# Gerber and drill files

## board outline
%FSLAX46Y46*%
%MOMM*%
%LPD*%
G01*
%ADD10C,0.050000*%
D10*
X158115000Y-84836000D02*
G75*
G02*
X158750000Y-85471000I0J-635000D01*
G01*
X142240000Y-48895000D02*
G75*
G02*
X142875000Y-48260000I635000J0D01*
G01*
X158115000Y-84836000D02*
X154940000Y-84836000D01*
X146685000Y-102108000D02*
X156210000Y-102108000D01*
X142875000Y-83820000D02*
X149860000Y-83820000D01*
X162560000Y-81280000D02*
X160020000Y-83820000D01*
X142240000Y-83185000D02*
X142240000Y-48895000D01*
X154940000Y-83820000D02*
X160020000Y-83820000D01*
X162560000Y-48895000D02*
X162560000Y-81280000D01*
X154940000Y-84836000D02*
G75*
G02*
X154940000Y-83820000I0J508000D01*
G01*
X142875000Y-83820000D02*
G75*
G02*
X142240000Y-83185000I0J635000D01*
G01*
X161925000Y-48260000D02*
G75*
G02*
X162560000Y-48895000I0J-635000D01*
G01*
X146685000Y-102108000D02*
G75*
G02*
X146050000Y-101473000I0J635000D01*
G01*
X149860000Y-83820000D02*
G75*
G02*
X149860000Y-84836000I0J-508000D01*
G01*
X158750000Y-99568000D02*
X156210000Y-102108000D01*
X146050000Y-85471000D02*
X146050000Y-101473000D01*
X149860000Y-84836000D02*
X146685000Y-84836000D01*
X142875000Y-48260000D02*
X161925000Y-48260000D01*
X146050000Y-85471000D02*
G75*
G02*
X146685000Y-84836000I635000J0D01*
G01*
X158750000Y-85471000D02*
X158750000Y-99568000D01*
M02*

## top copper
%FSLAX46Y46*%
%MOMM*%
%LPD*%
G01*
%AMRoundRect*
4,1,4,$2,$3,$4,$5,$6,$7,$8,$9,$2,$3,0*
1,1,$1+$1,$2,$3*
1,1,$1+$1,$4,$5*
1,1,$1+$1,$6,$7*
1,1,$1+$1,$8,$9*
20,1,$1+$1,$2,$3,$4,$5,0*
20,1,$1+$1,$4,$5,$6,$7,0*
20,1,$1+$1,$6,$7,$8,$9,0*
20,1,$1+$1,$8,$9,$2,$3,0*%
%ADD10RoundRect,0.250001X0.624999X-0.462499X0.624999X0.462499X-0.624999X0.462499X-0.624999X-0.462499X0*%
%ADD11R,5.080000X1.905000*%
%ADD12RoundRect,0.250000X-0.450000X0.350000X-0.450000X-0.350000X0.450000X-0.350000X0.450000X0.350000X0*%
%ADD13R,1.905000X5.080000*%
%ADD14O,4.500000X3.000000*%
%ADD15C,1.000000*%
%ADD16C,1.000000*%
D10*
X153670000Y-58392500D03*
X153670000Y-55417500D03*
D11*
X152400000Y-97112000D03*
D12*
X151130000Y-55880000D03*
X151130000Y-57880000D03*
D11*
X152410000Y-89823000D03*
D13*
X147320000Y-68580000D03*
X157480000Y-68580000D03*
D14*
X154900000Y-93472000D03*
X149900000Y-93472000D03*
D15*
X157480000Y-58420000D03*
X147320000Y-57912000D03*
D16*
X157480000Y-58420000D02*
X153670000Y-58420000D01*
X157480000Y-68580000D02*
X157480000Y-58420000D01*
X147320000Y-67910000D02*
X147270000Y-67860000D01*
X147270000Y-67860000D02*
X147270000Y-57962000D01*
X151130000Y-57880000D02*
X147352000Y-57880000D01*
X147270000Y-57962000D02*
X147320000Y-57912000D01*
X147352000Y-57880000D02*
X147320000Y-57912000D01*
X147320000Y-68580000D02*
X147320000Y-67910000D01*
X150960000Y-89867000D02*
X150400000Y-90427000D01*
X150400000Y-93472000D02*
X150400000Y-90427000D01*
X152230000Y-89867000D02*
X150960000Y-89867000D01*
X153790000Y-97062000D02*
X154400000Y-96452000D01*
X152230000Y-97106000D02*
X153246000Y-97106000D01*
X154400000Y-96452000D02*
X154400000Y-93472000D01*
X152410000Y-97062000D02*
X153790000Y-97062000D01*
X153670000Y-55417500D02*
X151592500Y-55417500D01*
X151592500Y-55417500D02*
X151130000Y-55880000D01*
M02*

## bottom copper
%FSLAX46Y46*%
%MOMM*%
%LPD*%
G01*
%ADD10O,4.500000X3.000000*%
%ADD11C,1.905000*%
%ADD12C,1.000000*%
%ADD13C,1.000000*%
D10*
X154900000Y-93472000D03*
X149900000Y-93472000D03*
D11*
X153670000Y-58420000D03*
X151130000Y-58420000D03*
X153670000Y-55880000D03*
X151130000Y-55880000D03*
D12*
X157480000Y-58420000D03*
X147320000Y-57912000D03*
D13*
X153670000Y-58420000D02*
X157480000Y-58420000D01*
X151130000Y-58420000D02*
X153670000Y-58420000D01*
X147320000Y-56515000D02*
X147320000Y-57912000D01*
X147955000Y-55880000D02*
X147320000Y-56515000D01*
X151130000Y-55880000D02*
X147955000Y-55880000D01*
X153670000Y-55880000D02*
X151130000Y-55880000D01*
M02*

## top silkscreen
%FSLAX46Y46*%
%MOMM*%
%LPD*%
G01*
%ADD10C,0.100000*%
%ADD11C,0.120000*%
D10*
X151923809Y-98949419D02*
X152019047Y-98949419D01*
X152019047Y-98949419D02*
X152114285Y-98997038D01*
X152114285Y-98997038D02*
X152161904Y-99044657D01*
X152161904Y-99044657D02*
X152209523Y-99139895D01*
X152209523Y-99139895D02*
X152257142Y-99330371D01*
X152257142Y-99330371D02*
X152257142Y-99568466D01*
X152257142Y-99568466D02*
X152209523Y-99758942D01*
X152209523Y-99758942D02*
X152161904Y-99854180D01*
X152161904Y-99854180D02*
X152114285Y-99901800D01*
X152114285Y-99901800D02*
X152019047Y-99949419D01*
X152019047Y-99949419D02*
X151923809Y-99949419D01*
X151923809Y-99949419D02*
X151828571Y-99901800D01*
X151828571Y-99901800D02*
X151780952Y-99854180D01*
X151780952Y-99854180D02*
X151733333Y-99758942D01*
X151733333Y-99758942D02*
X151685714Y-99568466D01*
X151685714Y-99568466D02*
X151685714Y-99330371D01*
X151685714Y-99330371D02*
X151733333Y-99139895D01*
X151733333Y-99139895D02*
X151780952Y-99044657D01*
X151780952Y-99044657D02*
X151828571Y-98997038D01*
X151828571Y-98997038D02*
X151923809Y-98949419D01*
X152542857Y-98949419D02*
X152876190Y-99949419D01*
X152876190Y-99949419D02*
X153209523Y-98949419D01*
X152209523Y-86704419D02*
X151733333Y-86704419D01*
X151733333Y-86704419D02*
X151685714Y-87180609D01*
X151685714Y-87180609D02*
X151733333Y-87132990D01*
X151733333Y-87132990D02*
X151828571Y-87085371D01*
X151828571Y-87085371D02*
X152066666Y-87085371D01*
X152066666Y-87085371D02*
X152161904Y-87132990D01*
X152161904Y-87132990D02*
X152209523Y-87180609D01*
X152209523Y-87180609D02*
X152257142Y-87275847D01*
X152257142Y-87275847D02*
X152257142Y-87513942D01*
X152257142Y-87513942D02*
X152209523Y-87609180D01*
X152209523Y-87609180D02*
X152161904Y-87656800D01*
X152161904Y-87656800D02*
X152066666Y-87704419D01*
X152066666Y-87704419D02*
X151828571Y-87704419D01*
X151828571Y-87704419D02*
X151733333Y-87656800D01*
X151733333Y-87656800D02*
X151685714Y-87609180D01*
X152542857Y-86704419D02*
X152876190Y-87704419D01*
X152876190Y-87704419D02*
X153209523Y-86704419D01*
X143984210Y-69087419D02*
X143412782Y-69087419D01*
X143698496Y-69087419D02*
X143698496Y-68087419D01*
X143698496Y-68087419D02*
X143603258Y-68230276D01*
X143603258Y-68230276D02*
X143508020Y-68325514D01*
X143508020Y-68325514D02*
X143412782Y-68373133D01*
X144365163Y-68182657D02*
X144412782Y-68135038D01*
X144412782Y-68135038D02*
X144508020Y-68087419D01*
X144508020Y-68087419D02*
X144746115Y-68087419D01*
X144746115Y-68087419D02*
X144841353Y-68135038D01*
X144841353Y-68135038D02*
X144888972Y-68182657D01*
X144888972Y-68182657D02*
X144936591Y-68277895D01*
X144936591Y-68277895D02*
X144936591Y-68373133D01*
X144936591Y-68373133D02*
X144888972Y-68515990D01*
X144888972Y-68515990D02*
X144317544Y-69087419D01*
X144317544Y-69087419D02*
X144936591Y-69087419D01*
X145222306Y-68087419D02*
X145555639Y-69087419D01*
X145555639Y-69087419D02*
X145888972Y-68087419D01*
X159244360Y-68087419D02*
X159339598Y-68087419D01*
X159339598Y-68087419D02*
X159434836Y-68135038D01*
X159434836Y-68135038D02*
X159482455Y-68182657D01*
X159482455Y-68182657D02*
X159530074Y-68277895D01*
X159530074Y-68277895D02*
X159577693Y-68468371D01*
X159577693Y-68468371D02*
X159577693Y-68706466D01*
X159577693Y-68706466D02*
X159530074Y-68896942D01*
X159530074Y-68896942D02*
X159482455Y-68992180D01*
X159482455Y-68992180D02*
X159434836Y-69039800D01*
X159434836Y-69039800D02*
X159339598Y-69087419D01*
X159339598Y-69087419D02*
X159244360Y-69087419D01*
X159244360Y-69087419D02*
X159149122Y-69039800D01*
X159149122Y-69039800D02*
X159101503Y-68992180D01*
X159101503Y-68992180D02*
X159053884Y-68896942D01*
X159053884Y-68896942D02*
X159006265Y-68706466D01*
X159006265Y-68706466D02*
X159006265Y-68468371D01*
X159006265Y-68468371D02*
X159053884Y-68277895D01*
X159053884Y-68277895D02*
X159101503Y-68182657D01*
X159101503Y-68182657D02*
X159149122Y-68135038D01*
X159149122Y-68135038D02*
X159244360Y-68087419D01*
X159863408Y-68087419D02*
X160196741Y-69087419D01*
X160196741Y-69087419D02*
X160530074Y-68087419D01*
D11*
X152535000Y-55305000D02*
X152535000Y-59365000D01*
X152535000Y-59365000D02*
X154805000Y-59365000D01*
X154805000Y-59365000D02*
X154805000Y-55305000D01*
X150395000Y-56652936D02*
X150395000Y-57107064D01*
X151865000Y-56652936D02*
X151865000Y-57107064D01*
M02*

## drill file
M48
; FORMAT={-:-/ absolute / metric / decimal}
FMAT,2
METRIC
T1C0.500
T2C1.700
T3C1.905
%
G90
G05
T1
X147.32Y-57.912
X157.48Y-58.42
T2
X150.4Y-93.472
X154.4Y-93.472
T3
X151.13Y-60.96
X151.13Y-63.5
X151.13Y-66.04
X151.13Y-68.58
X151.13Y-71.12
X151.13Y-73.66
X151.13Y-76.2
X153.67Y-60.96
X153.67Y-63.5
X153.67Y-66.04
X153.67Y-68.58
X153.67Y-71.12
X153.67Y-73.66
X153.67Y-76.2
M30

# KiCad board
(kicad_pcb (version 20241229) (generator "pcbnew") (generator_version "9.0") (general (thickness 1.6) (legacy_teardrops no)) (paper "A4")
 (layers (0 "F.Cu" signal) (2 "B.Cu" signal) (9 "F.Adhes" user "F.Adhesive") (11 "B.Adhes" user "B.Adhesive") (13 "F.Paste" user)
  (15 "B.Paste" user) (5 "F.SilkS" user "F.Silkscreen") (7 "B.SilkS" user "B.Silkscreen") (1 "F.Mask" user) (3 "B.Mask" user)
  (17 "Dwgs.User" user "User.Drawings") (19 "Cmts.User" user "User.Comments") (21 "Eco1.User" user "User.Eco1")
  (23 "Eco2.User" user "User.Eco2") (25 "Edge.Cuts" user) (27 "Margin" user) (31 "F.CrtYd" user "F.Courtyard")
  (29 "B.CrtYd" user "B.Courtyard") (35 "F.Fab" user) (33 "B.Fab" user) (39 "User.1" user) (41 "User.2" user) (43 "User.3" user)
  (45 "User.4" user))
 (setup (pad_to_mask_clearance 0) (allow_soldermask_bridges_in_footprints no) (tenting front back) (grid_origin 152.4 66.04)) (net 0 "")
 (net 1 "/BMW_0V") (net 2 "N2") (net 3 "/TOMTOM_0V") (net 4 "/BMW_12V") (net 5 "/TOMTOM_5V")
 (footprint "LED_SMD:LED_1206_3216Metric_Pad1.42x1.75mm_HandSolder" (layer "F.Cu") (at 153.67 56.905 90)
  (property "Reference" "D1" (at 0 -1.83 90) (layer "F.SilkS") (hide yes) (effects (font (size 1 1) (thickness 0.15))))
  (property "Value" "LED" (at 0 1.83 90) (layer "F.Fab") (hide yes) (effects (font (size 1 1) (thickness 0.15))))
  (fp_line (start 1.6 -1.135) (end -2.46 -1.135) (stroke (width 0.12) (type solid)) (layer "F.SilkS"))
  (fp_line (start -2.46 -1.135) (end -2.46 1.135) (stroke (width 0.12) (type solid)) (layer "F.SilkS"))
  (fp_line (start -2.46 1.135) (end 1.6 1.135) (stroke (width 0.12) (type solid)) (layer "F.SilkS"))
  (pad "1" smd roundrect (at -1.4875 0 90) (size 1.425 1.75) (layers "F.Cu" "F.Mask" "F.Paste") (roundrect_rratio 0.175439)
   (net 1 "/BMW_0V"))
  (pad "2" smd roundrect (at 1.4875 0 90) (size 1.425 1.75) (layers "F.Cu" "F.Mask" "F.Paste") (roundrect_rratio 0.175439) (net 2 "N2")))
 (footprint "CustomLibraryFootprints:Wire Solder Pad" (layer "F.Cu") (at 152.4 97.112 -90)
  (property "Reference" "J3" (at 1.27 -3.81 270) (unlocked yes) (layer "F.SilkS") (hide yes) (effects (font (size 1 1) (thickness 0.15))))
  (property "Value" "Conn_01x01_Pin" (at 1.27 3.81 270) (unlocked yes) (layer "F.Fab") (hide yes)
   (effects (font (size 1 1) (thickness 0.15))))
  (pad "1" smd rect (at 0 0 270) (size 1.905 5.08) (layers "F.Cu" "F.Mask" "F.Paste") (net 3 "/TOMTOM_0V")))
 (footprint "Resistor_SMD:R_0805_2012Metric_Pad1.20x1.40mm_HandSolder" (layer "F.Cu") (at 151.13 56.88 -90)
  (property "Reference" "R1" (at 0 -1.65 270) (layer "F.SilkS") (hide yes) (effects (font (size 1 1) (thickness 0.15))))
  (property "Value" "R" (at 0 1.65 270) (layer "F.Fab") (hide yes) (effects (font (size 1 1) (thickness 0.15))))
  (fp_line (start -0.227064 0.735) (end 0.227064 0.735) (stroke (width 0.12) (type solid)) (layer "F.SilkS"))
  (fp_line (start -0.227064 -0.735) (end 0.227064 -0.735) (stroke (width 0.12) (type solid)) (layer "F.SilkS"))
  (pad "1" smd roundrect (at -1 0 270) (size 1.2 1.4) (layers "F.Cu" "F.Mask" "F.Paste") (roundrect_rratio 0.208333) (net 2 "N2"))
  (pad "2" smd roundrect (at 1 0 270) (size 1.2 1.4) (layers "F.Cu" "F.Mask" "F.Paste") (roundrect_rratio 0.208333) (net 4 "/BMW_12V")))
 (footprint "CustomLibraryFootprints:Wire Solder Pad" (layer "F.Cu") (at 152.41 89.823 -90)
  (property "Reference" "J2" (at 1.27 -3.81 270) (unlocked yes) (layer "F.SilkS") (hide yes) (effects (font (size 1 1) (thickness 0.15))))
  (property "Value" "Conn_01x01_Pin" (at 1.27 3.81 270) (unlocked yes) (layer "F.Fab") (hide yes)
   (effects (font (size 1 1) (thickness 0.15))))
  (pad "1" smd rect (at 0 0 270) (size 1.905 5.08) (layers "F.Cu" "F.Mask" "F.Paste") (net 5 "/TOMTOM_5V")))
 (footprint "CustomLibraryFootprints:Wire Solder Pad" (layer "F.Cu") (at 147.32 68.58 180)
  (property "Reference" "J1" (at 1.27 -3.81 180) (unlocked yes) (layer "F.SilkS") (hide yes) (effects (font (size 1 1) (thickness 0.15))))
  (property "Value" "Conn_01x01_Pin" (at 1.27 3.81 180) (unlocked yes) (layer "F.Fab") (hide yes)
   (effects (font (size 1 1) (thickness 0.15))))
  (pad "1" smd rect (at 0 0 180) (size 1.905 5.08) (layers "F.Cu" "F.Mask" "F.Paste") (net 4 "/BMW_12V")))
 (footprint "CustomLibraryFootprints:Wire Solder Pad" (layer "F.Cu") (at 157.48 68.58 180)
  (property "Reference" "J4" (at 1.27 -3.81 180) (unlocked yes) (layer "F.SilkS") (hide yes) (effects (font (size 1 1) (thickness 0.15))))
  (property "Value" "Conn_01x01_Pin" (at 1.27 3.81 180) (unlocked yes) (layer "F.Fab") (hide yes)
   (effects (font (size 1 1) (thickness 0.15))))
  (pad "1" smd rect (at 0 0 180) (size 1.905 5.08) (layers "F.Cu" "F.Mask" "F.Paste") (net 1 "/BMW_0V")))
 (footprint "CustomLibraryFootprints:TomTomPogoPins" (layer "F.Cu") (at 154.4 93.472 180)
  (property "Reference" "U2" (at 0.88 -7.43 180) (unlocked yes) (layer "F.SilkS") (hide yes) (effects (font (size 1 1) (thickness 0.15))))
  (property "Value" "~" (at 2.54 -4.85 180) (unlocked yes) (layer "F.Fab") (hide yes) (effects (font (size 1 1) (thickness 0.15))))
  (pad "1" thru_hole oval (at 0 0 180) (size 4.5 3) (drill 1.7 (offset -0.5 0)) (layers "*.Cu" "*.Mask") (remove_unused_layers no)
   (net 3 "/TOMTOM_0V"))
  (pad "2" thru_hole oval (at 4 0 180) (size 4.5 3) (drill 1.7 (offset 0.5 0)) (layers "*.Cu" "*.Mask") (remove_unused_layers no)
   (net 5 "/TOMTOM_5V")))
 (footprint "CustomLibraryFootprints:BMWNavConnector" (layer "B.Cu") (at 151.13 76.2 180)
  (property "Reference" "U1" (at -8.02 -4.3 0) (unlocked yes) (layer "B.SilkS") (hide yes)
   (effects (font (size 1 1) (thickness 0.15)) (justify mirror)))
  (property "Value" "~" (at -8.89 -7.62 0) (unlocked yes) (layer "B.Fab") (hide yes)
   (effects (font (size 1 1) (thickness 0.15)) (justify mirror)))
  (pad "" np_thru_hole circle (at -2.54 0 180) (size 1.905 1.905) (drill 1.905) (layers "*.Cu" "*.Mask"))
  (pad "" np_thru_hole circle (at -2.54 2.54 180) (size 1.905 1.905) (drill 1.905) (layers "*.Cu" "*.Mask"))
  (pad "" np_thru_hole circle (at -2.54 5.08 180) (size 1.905 1.905) (drill 1.905) (layers "*.Cu" "*.Mask"))
  (pad "" np_thru_hole circle (at -2.54 7.62 180) (size 1.905 1.905) (drill 1.905) (layers "*.Cu" "*.Mask"))
  (pad "" np_thru_hole circle (at -2.54 10.16 180) (size 1.905 1.905) (drill 1.905) (layers "*.Cu" "*.Mask"))
  (pad "" np_thru_hole circle (at -2.54 12.7 180) (size 1.905 1.905) (drill 1.905) (layers "*.Cu" "*.Mask"))
  (pad "" np_thru_hole circle (at -2.54 15.24 180) (size 1.905 1.905) (drill 1.905) (layers "*.Cu" "*.Mask"))
  (pad "" np_thru_hole circle (at 0 0 180) (size 1.905 1.905) (drill 1.905) (layers "*.Cu" "*.Mask"))
  (pad "" np_thru_hole circle (at 0 2.54 180) (size 1.905 1.905) (drill 1.905) (layers "*.Cu" "*.Mask"))
  (pad "" np_thru_hole circle (at 0 5.08 180) (size 1.905 1.905) (drill 1.905) (layers "*.Cu" "*.Mask"))
  (pad "" np_thru_hole circle (at 0 7.62 180) (size 1.905 1.905) (drill 1.905) (layers "*.Cu" "*.Mask"))
  (pad "" np_thru_hole circle (at 0 10.16 180) (size 1.905 1.905) (drill 1.905) (layers "*.Cu" "*.Mask"))
  (pad "" np_thru_hole circle (at 0 12.7 180) (size 1.905 1.905) (drill 1.905) (layers "*.Cu" "*.Mask"))
  (pad "" np_thru_hole circle (at 0 15.24 180) (size 1.905 1.905) (drill 1.905) (layers "*.Cu" "*.Mask"))
  (pad "15" smd circle (at -2.54 17.78 180) (size 1.905 1.905) (layers "B.Cu" "B.Mask" "B.Paste") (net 1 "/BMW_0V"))
  (pad "16" smd circle (at 0 17.78 180) (size 1.905 1.905) (layers "B.Cu" "B.Mask" "B.Paste") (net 1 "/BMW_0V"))
  (pad "17" smd circle (at -2.54 20.32 180) (size 1.905 1.905) (layers "B.Cu" "B.Mask" "B.Paste") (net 4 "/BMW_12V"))
  (pad "18" smd circle (at 0 20.32 180) (size 1.905 1.905) (layers "B.Cu" "B.Mask" "B.Paste") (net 4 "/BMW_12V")))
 (gr_arc (start 158.115 84.836) (mid 158.564013 85.021987) (end 158.75 85.471) (stroke (width 0.05) (type default)) (layer "Edge.Cuts"))
 (gr_arc (start 142.24 48.895) (mid 142.425987 48.445987) (end 142.875 48.26) (stroke (width 0.05) (type default)) (layer "Edge.Cuts"))
 (gr_line (start 158.115 84.836) (end 154.94 84.836) (stroke (width 0.05) (type default)) (layer "Edge.Cuts"))
 (gr_line (start 146.685 102.108) (end 156.21 102.108) (stroke (width 0.05) (type default)) (layer "Edge.Cuts"))
 (gr_line (start 142.875 83.82) (end 149.86 83.82) (stroke (width 0.05) (type default)) (layer "Edge.Cuts"))
 (gr_line (start 162.56 81.28) (end 160.02 83.82) (stroke (width 0.05) (type default)) (layer "Edge.Cuts"))
 (gr_line (start 142.24 83.185) (end 142.24 48.895) (stroke (width 0.05) (type default)) (layer "Edge.Cuts"))
 (gr_line (start 154.94 83.82) (end 160.02 83.82) (stroke (width 0.05) (type default)) (layer "Edge.Cuts"))
 (gr_line (start 162.56 48.895) (end 162.56 81.28) (stroke (width 0.05) (type default)) (layer "Edge.Cuts"))
 (gr_arc (start 154.94 84.836) (mid 154.432 84.328) (end 154.94 83.82) (stroke (width 0.05) (type default)) (layer "Edge.Cuts"))
 (gr_arc (start 142.875 83.82) (mid 142.425987 83.634013) (end 142.24 83.185) (stroke (width 0.05) (type default)) (layer "Edge.Cuts"))
 (gr_arc (start 161.925 48.26) (mid 162.374013 48.445987) (end 162.56 48.895) (stroke (width 0.05) (type default)) (layer "Edge.Cuts"))
 (gr_arc (start 146.685 102.108) (mid 146.235987 101.922013) (end 146.05 101.473) (stroke (width 0.05) (type default)) (layer "Edge.Cuts"))
 (gr_arc (start 149.86 83.82) (mid 150.368 84.328) (end 149.86 84.836) (stroke (width 0.05) (type default)) (layer "Edge.Cuts"))
 (gr_line (start 158.75 99.568) (end 156.21 102.108) (stroke (width 0.05) (type default)) (layer "Edge.Cuts"))
 (gr_line (start 146.05 85.471) (end 146.05 101.473) (stroke (width 0.05) (type default)) (layer "Edge.Cuts"))
 (gr_line (start 149.86 84.836) (end 146.685 84.836) (stroke (width 0.05) (type default)) (layer "Edge.Cuts"))
 (gr_line (start 142.875 48.26) (end 161.925 48.26) (stroke (width 0.05) (type default)) (layer "Edge.Cuts"))
 (gr_arc (start 146.05 85.471) (mid 146.235987 85.021987) (end 146.685 84.836) (stroke (width 0.05) (type default)) (layer "Edge.Cuts"))
 (gr_line (start 158.75 85.471) (end 158.75 99.568) (stroke (width 0.05) (type default)) (layer "Edge.Cuts"))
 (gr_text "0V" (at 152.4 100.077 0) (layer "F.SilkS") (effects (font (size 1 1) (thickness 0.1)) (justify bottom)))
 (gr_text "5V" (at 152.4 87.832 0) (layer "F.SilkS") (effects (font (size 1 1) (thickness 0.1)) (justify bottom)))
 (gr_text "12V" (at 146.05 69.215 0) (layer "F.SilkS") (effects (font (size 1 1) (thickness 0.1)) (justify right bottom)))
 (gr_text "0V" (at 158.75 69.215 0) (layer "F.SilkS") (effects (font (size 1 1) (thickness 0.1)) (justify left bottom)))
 (segment (start 157.48 58.42) (end 153.67 58.42) (width 1) (layer "F.Cu") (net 1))
 (segment (start 157.48 68.58) (end 157.48 58.42) (width 1) (layer "F.Cu") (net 1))
 (via (at 157.48 58.42) (size 1) (drill 0.5) (layers "F.Cu" "B.Cu") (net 1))
 (segment (start 153.67 58.42) (end 157.48 58.42) (width 1) (layer "B.Cu") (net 1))
 (segment (start 151.13 58.42) (end 153.67 58.42) (width 1) (layer "B.Cu") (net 1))
 (segment (start 147.32 67.91) (end 147.27 67.86) (width 1) (layer "F.Cu") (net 4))
 (segment (start 147.27 67.86) (end 147.27 57.962) (width 1) (layer "F.Cu") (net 4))
 (segment (start 151.13 57.88) (end 147.352 57.88) (width 1) (layer "F.Cu") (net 4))
 (segment (start 147.27 57.962) (end 147.32 57.912) (width 1) (layer "F.Cu") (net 4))
 (segment (start 147.352 57.88) (end 147.32 57.912) (width 1) (layer "F.Cu") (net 4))
 (segment (start 147.32 68.58) (end 147.32 67.91) (width 1) (layer "F.Cu") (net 4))
 (via (at 147.32 57.912) (size 1) (drill 0.5) (layers "F.Cu" "B.Cu") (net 4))
 (segment (start 147.32 56.515) (end 147.32 57.912) (width 1) (layer "B.Cu") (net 4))
 (segment (start 147.955 55.88) (end 147.32 56.515) (width 1) (layer "B.Cu") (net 4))
 (segment (start 151.13 55.88) (end 147.955 55.88) (width 1) (layer "B.Cu") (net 4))
 (segment (start 153.67 55.88) (end 151.13 55.88) (width 1) (layer "B.Cu") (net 4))
 (segment (start 150.96 89.867) (end 150.4 90.427) (width 1) (layer "F.Cu") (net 5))
 (segment (start 150.4 93.472) (end 150.4 90.427) (width 1) (layer "F.Cu") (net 5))
 (segment (start 152.23 89.867) (end 150.96 89.867) (width 1) (layer "F.Cu") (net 5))
 (segment (start 153.79 97.062) (end 154.4 96.452) (width 1) (layer "F.Cu") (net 3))
 (segment (start 152.23 97.106) (end 153.246 97.106) (width 1) (layer "F.Cu") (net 3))
 (segment (start 154.4 96.452) (end 154.4 93.472) (width 1) (layer "F.Cu") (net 3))
 (segment (start 152.41 97.062) (end 153.79 97.062) (width 1) (layer "F.Cu") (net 3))
 (segment (start 153.67 55.4175) (end 151.5925 55.4175) (width 1) (layer "F.Cu") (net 2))
 (segment (start 151.5925 55.4175) (end 151.13 55.88) (width 1) (layer "F.Cu") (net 2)))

